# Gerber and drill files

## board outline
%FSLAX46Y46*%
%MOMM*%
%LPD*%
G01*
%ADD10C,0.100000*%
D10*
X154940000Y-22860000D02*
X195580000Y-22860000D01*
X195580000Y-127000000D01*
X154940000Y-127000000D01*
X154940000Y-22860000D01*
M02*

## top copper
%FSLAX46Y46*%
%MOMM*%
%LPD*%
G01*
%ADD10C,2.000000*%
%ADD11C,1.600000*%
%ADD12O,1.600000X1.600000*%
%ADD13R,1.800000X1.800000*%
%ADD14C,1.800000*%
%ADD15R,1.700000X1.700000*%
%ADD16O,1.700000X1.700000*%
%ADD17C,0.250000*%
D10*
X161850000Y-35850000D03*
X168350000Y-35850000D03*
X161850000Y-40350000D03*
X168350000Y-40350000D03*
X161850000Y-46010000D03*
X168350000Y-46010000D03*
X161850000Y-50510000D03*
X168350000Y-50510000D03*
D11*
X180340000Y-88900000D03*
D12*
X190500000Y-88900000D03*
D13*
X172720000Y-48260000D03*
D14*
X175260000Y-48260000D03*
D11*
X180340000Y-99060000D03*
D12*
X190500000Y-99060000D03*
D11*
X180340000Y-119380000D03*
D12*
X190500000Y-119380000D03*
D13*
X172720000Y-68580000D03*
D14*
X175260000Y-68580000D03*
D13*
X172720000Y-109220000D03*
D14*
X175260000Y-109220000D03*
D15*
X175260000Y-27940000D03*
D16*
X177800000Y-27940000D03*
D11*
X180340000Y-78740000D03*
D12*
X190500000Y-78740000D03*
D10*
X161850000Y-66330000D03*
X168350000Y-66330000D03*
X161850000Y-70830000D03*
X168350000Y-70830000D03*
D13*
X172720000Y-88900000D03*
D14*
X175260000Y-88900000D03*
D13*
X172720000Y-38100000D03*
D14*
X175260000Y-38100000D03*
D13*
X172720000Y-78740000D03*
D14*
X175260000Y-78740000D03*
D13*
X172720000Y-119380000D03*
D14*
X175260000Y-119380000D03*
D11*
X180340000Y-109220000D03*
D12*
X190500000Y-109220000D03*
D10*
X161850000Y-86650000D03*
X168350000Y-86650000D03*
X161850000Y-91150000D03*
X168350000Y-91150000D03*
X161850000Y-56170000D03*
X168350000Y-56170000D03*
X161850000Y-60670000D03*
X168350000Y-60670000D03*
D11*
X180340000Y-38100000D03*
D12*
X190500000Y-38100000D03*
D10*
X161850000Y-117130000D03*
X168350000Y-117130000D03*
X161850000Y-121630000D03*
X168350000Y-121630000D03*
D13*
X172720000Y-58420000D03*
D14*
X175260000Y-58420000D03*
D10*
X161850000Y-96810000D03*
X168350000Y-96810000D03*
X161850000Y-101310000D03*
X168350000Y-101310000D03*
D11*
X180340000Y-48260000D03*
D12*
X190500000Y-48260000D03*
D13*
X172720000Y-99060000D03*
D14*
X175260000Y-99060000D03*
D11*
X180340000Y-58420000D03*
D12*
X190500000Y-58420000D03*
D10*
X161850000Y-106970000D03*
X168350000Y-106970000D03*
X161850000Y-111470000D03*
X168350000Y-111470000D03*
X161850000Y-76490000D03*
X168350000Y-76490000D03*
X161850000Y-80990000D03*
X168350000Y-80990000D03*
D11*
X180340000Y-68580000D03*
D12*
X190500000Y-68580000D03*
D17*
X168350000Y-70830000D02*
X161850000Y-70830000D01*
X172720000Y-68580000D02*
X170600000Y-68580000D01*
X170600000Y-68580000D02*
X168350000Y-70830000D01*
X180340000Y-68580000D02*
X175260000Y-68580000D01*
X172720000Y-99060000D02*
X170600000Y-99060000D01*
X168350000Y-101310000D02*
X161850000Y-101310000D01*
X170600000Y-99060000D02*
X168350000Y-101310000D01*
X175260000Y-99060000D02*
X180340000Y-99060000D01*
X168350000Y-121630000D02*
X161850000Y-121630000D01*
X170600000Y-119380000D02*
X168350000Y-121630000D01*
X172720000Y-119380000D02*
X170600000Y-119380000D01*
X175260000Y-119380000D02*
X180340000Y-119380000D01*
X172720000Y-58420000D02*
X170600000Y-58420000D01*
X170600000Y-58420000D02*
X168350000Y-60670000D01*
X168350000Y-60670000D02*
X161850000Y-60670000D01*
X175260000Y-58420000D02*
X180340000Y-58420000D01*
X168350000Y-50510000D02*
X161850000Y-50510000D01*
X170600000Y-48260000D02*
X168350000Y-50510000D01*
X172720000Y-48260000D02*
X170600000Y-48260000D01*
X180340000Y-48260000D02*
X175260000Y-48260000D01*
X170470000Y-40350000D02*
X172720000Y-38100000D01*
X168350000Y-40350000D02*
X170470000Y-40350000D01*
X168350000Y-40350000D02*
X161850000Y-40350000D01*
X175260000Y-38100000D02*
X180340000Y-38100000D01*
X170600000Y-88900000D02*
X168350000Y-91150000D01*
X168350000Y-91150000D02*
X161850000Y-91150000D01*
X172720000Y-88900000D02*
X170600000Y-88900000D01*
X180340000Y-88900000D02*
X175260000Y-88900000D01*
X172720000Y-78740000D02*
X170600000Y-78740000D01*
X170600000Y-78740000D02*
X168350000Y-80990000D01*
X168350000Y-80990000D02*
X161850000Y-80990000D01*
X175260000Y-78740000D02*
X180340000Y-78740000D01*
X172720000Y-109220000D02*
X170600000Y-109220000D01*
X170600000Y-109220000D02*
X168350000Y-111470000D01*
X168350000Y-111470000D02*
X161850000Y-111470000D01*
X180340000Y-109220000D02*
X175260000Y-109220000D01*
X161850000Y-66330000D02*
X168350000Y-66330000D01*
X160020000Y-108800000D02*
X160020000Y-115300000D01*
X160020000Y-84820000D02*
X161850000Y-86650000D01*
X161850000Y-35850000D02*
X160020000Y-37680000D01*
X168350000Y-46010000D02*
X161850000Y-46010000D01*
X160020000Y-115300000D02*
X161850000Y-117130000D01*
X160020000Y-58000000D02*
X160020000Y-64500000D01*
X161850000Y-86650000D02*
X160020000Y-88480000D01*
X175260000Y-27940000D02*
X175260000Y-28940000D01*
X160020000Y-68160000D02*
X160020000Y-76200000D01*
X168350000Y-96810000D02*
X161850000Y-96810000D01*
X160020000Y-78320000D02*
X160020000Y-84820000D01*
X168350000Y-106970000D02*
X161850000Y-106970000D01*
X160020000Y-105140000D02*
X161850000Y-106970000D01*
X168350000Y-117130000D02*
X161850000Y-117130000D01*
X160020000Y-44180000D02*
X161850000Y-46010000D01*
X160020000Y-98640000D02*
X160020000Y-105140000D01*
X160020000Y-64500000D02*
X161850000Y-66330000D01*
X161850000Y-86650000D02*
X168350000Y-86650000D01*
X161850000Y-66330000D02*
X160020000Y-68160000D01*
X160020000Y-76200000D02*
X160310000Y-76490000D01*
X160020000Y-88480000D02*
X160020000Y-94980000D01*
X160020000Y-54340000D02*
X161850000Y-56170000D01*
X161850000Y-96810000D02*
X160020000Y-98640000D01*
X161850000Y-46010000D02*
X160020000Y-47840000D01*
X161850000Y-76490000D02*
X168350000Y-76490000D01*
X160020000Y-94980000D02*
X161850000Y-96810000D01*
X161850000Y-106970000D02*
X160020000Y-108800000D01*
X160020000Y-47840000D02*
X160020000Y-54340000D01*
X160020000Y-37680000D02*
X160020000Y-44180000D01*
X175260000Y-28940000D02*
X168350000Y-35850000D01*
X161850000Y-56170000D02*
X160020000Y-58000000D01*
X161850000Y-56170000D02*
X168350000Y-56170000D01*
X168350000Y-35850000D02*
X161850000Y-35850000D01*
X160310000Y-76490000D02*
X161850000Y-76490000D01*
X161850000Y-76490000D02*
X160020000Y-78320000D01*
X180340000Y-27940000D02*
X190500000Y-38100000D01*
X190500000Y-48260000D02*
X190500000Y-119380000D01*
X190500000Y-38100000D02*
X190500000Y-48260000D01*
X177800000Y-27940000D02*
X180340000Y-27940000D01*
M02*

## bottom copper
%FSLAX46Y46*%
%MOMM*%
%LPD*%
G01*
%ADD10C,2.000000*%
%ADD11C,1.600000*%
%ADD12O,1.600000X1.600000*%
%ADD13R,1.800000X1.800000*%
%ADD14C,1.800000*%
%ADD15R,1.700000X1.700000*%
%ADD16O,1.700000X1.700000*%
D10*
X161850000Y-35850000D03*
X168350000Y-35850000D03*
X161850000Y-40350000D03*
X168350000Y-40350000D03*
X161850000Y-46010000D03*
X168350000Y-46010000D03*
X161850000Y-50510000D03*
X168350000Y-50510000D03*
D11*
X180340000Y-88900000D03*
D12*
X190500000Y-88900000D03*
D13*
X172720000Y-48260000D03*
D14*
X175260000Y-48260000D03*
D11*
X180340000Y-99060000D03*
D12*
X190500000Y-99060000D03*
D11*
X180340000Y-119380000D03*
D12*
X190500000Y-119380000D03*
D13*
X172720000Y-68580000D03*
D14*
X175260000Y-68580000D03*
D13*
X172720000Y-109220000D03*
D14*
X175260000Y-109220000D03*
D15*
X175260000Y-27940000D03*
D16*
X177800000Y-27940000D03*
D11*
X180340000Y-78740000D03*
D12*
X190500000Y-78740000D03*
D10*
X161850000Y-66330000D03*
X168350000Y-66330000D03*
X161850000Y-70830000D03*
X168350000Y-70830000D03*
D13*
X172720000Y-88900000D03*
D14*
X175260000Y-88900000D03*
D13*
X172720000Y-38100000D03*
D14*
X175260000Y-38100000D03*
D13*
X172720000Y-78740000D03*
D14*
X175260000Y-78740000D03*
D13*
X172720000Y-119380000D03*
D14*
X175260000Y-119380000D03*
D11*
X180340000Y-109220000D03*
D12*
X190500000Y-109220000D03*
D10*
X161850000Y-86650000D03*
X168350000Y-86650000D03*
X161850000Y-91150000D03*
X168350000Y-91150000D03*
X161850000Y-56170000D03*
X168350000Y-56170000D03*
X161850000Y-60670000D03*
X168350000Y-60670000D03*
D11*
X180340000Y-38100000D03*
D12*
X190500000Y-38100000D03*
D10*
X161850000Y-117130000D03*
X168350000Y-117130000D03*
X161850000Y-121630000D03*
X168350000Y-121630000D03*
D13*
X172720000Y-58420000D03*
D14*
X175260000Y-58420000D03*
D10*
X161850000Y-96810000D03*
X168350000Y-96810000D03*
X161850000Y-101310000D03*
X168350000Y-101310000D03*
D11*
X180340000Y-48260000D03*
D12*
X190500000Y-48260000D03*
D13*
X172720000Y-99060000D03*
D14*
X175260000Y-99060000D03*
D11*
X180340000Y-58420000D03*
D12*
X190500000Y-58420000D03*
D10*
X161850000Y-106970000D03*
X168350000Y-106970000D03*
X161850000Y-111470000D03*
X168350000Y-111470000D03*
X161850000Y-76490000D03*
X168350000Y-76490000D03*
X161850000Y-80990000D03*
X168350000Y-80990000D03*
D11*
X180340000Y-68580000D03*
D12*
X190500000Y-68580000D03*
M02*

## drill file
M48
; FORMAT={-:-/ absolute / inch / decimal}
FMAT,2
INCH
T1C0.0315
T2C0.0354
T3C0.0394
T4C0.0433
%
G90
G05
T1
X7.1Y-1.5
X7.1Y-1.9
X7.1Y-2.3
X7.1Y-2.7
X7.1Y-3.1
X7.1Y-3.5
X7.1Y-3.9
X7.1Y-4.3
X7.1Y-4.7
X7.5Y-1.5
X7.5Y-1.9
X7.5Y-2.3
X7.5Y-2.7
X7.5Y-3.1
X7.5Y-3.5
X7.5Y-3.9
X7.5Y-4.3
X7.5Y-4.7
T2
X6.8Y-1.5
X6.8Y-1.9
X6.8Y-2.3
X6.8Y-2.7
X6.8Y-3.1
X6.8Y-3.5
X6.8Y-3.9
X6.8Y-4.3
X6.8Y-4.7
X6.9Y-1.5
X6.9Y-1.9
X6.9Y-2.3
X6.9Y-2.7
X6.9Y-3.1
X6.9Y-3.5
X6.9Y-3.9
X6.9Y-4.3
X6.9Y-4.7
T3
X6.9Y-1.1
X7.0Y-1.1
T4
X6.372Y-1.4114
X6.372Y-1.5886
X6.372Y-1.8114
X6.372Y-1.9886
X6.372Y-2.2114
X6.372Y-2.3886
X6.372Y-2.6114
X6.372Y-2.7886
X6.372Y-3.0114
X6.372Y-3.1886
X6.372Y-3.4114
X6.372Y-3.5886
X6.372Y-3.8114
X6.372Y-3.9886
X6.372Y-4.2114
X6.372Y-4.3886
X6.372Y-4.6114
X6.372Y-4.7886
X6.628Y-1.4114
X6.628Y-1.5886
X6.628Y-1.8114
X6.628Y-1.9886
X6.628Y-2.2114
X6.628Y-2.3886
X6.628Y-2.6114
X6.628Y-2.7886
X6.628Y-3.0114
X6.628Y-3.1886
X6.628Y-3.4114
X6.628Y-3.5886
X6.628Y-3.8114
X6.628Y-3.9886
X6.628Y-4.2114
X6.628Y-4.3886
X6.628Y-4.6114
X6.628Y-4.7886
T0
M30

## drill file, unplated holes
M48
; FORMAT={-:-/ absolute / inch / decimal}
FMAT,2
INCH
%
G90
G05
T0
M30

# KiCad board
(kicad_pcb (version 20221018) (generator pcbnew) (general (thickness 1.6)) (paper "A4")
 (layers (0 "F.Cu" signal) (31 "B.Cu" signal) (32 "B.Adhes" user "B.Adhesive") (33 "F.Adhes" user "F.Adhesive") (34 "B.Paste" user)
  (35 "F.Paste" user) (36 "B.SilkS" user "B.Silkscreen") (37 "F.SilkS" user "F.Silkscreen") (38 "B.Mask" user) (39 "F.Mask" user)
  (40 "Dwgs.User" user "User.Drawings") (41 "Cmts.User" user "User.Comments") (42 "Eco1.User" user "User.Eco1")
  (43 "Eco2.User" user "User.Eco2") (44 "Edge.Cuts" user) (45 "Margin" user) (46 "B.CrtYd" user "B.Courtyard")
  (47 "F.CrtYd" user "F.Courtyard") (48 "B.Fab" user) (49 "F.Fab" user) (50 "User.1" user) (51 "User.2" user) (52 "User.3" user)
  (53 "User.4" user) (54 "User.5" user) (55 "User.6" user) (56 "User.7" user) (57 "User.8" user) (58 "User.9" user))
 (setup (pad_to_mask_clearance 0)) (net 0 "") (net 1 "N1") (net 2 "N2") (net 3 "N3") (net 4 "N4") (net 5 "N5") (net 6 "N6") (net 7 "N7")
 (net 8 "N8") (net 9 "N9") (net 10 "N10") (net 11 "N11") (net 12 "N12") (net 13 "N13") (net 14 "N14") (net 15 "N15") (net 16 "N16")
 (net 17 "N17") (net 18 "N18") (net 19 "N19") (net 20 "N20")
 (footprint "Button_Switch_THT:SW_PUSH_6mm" (layer "F.Cu") (at 161.85 35.85)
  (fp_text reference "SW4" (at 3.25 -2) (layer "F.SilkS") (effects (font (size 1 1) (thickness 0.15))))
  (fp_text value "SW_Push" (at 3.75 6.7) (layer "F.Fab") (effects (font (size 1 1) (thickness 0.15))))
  (pad "1" thru_hole circle (at 0 0 90) (size 2 2) (drill 1.1) (layers "*.Cu" "*.Mask") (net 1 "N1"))
  (pad "1" thru_hole circle (at 6.5 0 90) (size 2 2) (drill 1.1) (layers "*.Cu" "*.Mask") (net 1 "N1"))
  (pad "2" thru_hole circle (at 0 4.5 90) (size 2 2) (drill 1.1) (layers "*.Cu" "*.Mask") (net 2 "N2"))
  (pad "2" thru_hole circle (at 6.5 4.5 90) (size 2 2) (drill 1.1) (layers "*.Cu" "*.Mask") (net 2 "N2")))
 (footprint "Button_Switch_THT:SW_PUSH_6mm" (layer "F.Cu") (at 161.85 46.01)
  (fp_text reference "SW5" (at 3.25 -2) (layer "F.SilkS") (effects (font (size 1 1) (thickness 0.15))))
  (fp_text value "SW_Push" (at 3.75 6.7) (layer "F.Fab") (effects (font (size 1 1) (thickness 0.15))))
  (pad "1" thru_hole circle (at 0 0 90) (size 2 2) (drill 1.1) (layers "*.Cu" "*.Mask") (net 1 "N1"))
  (pad "1" thru_hole circle (at 6.5 0 90) (size 2 2) (drill 1.1) (layers "*.Cu" "*.Mask") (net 1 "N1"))
  (pad "2" thru_hole circle (at 0 4.5 90) (size 2 2) (drill 1.1) (layers "*.Cu" "*.Mask") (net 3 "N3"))
  (pad "2" thru_hole circle (at 6.5 4.5 90) (size 2 2) (drill 1.1) (layers "*.Cu" "*.Mask") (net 3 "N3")))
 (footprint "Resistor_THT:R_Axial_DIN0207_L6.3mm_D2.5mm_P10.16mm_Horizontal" (layer "F.Cu") (at 180.34 88.9)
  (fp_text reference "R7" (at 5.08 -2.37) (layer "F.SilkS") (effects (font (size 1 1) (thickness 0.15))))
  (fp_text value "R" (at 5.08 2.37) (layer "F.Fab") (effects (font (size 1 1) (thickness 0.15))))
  (pad "1" thru_hole circle (at 0 0) (size 1.6 1.6) (drill 0.8) (layers "*.Cu" "*.Mask") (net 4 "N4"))
  (pad "2" thru_hole oval (at 10.16 0) (size 1.6 1.6) (drill 0.8) (layers "*.Cu" "*.Mask") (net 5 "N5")))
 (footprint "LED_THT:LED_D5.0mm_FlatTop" (layer "F.Cu") (at 172.72 48.26)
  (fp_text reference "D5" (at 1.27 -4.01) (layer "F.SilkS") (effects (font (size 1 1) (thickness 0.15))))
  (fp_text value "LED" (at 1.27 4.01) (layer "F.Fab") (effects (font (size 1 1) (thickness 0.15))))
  (pad "1" thru_hole rect (at 0 0) (size 1.8 1.8) (drill 0.9) (layers "*.Cu" "*.Mask") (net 3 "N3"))
  (pad "2" thru_hole circle (at 2.54 0) (size 1.8 1.8) (drill 0.9) (layers "*.Cu" "*.Mask") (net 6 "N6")))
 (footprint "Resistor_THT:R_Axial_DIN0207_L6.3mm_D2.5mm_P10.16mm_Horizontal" (layer "F.Cu") (at 180.34 99.06)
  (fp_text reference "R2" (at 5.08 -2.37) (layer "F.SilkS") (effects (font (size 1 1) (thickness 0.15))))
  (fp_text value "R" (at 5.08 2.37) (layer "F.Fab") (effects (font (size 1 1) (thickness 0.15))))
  (pad "1" thru_hole circle (at 0 0) (size 1.6 1.6) (drill 0.8) (layers "*.Cu" "*.Mask") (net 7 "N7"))
  (pad "2" thru_hole oval (at 10.16 0) (size 1.6 1.6) (drill 0.8) (layers "*.Cu" "*.Mask") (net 5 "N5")))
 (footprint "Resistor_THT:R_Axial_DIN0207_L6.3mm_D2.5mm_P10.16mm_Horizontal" (layer "F.Cu") (at 180.34 119.38)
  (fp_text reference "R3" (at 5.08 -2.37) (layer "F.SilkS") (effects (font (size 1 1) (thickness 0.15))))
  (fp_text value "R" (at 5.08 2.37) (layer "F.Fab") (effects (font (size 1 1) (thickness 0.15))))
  (pad "1" thru_hole circle (at 0 0) (size 1.6 1.6) (drill 0.8) (layers "*.Cu" "*.Mask") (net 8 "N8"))
  (pad "2" thru_hole oval (at 10.16 0) (size 1.6 1.6) (drill 0.8) (layers "*.Cu" "*.Mask") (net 5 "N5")))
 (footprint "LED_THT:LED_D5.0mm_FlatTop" (layer "F.Cu") (at 172.72 68.58)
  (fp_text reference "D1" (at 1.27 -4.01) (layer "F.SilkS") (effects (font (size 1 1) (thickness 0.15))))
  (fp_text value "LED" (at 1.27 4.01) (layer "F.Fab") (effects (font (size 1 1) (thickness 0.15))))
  (pad "1" thru_hole rect (at 0 0) (size 1.8 1.8) (drill 0.9) (layers "*.Cu" "*.Mask") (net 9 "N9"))
  (pad "2" thru_hole circle (at 2.54 0) (size 1.8 1.8) (drill 0.9) (layers "*.Cu" "*.Mask") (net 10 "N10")))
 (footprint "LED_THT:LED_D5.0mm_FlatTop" (layer "F.Cu") (at 172.72 109.22)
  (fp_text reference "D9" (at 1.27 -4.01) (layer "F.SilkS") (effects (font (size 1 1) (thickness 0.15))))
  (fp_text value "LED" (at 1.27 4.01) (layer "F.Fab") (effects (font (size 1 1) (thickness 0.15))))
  (pad "1" thru_hole rect (at 0 0) (size 1.8 1.8) (drill 0.9) (layers "*.Cu" "*.Mask") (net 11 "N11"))
  (pad "2" thru_hole circle (at 2.54 0) (size 1.8 1.8) (drill 0.9) (layers "*.Cu" "*.Mask") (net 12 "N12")))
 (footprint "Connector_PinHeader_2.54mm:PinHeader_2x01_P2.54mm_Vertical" (layer "F.Cu") (at 175.26 27.94)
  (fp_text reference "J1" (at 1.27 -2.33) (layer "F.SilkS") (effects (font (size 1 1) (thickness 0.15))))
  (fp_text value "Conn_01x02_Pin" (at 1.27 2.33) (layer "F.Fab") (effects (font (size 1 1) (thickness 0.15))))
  (pad "1" thru_hole rect (at 0 0) (size 1.7 1.7) (drill 1) (layers "*.Cu" "*.Mask") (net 1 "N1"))
  (pad "2" thru_hole oval (at 2.54 0) (size 1.7 1.7) (drill 1) (layers "*.Cu" "*.Mask") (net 5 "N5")))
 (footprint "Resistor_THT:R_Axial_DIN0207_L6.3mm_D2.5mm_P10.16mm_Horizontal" (layer "F.Cu") (at 180.34 78.74)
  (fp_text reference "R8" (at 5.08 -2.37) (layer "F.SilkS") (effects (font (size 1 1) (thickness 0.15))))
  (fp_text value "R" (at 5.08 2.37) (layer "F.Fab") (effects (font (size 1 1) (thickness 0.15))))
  (pad "1" thru_hole circle (at 0 0) (size 1.6 1.6) (drill 0.8) (layers "*.Cu" "*.Mask") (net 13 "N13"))
  (pad "2" thru_hole oval (at 10.16 0) (size 1.6 1.6) (drill 0.8) (layers "*.Cu" "*.Mask") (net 5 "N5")))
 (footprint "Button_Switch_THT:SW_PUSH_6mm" (layer "F.Cu") (at 161.85 66.33)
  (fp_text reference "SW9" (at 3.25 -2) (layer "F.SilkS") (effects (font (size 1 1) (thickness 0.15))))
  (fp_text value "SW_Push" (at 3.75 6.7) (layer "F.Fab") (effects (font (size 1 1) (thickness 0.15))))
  (pad "1" thru_hole circle (at 0 0 90) (size 2 2) (drill 1.1) (layers "*.Cu" "*.Mask") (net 1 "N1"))
  (pad "1" thru_hole circle (at 6.5 0 90) (size 2 2) (drill 1.1) (layers "*.Cu" "*.Mask") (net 1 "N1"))
  (pad "2" thru_hole circle (at 0 4.5 90) (size 2 2) (drill 1.1) (layers "*.Cu" "*.Mask") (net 9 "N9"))
  (pad "2" thru_hole circle (at 6.5 4.5 90) (size 2 2) (drill 1.1) (layers "*.Cu" "*.Mask") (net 9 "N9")))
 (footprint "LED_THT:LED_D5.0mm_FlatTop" (layer "F.Cu") (at 172.72 88.9)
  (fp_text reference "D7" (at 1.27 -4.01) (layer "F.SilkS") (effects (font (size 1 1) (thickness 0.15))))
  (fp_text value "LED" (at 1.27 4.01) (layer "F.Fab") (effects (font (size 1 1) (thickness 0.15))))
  (pad "1" thru_hole rect (at 0 0) (size 1.8 1.8) (drill 0.9) (layers "*.Cu" "*.Mask") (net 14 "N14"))
  (pad "2" thru_hole circle (at 2.54 0) (size 1.8 1.8) (drill 0.9) (layers "*.Cu" "*.Mask") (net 4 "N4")))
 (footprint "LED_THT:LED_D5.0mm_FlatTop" (layer "F.Cu") (at 172.72 38.1)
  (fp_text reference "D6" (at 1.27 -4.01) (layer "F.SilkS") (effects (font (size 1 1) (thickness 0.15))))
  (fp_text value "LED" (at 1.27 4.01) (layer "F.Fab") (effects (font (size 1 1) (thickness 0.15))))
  (pad "1" thru_hole rect (at 0 0) (size 1.8 1.8) (drill 0.9) (layers "*.Cu" "*.Mask") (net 2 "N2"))
  (pad "2" thru_hole circle (at 2.54 0) (size 1.8 1.8) (drill 0.9) (layers "*.Cu" "*.Mask") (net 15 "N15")))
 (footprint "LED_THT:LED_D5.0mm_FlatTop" (layer "F.Cu") (at 172.72 78.74)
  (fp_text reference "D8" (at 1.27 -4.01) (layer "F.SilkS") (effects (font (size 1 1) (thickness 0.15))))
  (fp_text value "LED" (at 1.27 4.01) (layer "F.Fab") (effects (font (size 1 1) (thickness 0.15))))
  (pad "1" thru_hole rect (at 0 0) (size 1.8 1.8) (drill 0.9) (layers "*.Cu" "*.Mask") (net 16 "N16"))
  (pad "2" thru_hole circle (at 2.54 0) (size 1.8 1.8) (drill 0.9) (layers "*.Cu" "*.Mask") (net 13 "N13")))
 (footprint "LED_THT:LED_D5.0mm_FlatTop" (layer "F.Cu") (at 172.72 119.38)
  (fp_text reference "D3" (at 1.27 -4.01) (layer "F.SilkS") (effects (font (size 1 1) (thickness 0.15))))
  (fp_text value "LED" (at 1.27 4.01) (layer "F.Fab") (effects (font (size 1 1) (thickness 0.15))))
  (pad "1" thru_hole rect (at 0 0) (size 1.8 1.8) (drill 0.9) (layers "*.Cu" "*.Mask") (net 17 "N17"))
  (pad "2" thru_hole circle (at 2.54 0) (size 1.8 1.8) (drill 0.9) (layers "*.Cu" "*.Mask") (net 8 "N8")))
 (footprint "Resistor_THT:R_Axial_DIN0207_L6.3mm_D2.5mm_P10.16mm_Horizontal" (layer "F.Cu") (at 180.34 109.22)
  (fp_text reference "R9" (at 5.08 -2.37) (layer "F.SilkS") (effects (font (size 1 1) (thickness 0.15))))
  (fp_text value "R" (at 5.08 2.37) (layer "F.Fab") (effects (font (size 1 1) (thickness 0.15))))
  (pad "1" thru_hole circle (at 0 0) (size 1.6 1.6) (drill 0.8) (layers "*.Cu" "*.Mask") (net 12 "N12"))
  (pad "2" thru_hole oval (at 10.16 0) (size 1.6 1.6) (drill 0.8) (layers "*.Cu" "*.Mask") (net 5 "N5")))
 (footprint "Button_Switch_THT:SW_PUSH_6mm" (layer "F.Cu") (at 161.85 86.65)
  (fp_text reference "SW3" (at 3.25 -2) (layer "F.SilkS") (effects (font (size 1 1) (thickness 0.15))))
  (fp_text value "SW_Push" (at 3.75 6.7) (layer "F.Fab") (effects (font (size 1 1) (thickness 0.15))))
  (pad "1" thru_hole circle (at 0 0 90) (size 2 2) (drill 1.1) (layers "*.Cu" "*.Mask") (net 1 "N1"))
  (pad "1" thru_hole circle (at 6.5 0 90) (size 2 2) (drill 1.1) (layers "*.Cu" "*.Mask") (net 1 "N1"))
  (pad "2" thru_hole circle (at 0 4.5 90) (size 2 2) (drill 1.1) (layers "*.Cu" "*.Mask") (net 14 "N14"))
  (pad "2" thru_hole circle (at 6.5 4.5 90) (size 2 2) (drill 1.1) (layers "*.Cu" "*.Mask") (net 14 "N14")))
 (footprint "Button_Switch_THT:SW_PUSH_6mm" (layer "F.Cu") (at 161.85 56.17)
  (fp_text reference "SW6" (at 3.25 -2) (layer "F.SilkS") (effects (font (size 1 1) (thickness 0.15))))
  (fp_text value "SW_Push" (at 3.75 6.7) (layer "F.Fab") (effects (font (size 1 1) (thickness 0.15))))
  (pad "1" thru_hole circle (at 0 0 90) (size 2 2) (drill 1.1) (layers "*.Cu" "*.Mask") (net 1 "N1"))
  (pad "1" thru_hole circle (at 6.5 0 90) (size 2 2) (drill 1.1) (layers "*.Cu" "*.Mask") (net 1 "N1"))
  (pad "2" thru_hole circle (at 0 4.5 90) (size 2 2) (drill 1.1) (layers "*.Cu" "*.Mask") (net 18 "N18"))
  (pad "2" thru_hole circle (at 6.5 4.5 90) (size 2 2) (drill 1.1) (layers "*.Cu" "*.Mask") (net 18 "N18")))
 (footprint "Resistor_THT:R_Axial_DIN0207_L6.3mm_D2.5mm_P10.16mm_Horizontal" (layer "F.Cu") (at 180.34 38.1)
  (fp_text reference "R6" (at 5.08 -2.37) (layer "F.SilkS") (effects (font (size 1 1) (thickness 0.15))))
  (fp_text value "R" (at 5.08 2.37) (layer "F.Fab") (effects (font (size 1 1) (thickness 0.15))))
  (pad "1" thru_hole circle (at 0 0) (size 1.6 1.6) (drill 0.8) (layers "*.Cu" "*.Mask") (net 15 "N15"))
  (pad "2" thru_hole oval (at 10.16 0) (size 1.6 1.6) (drill 0.8) (layers "*.Cu" "*.Mask") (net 5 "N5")))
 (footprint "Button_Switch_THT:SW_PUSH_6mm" (layer "F.Cu") (at 161.85 117.13)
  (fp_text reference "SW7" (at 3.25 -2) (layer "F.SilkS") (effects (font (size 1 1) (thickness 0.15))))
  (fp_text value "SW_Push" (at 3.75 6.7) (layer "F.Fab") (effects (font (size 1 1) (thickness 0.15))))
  (pad "1" thru_hole circle (at 0 0 90) (size 2 2) (drill 1.1) (layers "*.Cu" "*.Mask") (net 1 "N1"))
  (pad "1" thru_hole circle (at 6.5 0 90) (size 2 2) (drill 1.1) (layers "*.Cu" "*.Mask") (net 1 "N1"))
  (pad "2" thru_hole circle (at 0 4.5 90) (size 2 2) (drill 1.1) (layers "*.Cu" "*.Mask") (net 17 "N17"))
  (pad "2" thru_hole circle (at 6.5 4.5 90) (size 2 2) (drill 1.1) (layers "*.Cu" "*.Mask") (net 17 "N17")))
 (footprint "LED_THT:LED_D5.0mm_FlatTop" (layer "F.Cu") (at 172.72 58.42)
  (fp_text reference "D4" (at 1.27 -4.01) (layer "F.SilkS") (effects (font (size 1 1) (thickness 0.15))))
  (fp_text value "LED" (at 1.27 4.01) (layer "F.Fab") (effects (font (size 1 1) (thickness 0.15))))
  (pad "1" thru_hole rect (at 0 0) (size 1.8 1.8) (drill 0.9) (layers "*.Cu" "*.Mask") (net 18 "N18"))
  (pad "2" thru_hole circle (at 2.54 0) (size 1.8 1.8) (drill 0.9) (layers "*.Cu" "*.Mask") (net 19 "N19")))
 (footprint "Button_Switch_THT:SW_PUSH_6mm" (layer "F.Cu") (at 161.85 96.81)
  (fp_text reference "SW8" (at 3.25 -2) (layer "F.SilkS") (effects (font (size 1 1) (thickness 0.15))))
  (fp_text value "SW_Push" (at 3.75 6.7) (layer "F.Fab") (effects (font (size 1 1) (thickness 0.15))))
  (pad "1" thru_hole circle (at 0 0 90) (size 2 2) (drill 1.1) (layers "*.Cu" "*.Mask") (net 1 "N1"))
  (pad "1" thru_hole circle (at 6.5 0 90) (size 2 2) (drill 1.1) (layers "*.Cu" "*.Mask") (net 1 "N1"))
  (pad "2" thru_hole circle (at 0 4.5 90) (size 2 2) (drill 1.1) (layers "*.Cu" "*.Mask") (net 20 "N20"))
  (pad "2" thru_hole circle (at 6.5 4.5 90) (size 2 2) (drill 1.1) (layers "*.Cu" "*.Mask") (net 20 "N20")))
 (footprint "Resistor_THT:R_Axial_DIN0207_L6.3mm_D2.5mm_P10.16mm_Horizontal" (layer "F.Cu") (at 180.34 48.26)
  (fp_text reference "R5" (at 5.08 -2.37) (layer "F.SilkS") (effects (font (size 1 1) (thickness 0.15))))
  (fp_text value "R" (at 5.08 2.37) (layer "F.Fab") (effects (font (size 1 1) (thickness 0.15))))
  (pad "1" thru_hole circle (at 0 0) (size 1.6 1.6) (drill 0.8) (layers "*.Cu" "*.Mask") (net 6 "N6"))
  (pad "2" thru_hole oval (at 10.16 0) (size 1.6 1.6) (drill 0.8) (layers "*.Cu" "*.Mask") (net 5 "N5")))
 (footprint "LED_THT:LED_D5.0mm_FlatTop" (layer "F.Cu") (at 172.72 99.06)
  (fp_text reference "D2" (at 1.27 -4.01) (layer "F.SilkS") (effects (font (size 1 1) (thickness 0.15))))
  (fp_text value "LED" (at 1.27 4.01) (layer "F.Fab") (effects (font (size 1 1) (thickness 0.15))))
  (pad "1" thru_hole rect (at 0 0) (size 1.8 1.8) (drill 0.9) (layers "*.Cu" "*.Mask") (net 20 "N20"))
  (pad "2" thru_hole circle (at 2.54 0) (size 1.8 1.8) (drill 0.9) (layers "*.Cu" "*.Mask") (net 7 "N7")))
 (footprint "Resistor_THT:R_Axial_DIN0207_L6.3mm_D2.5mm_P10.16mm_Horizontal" (layer "F.Cu") (at 180.34 58.42)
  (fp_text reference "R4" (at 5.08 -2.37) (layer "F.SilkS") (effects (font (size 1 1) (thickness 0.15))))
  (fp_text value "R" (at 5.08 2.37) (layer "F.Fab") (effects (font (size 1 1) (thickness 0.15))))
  (pad "1" thru_hole circle (at 0 0) (size 1.6 1.6) (drill 0.8) (layers "*.Cu" "*.Mask") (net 19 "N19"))
  (pad "2" thru_hole oval (at 10.16 0) (size 1.6 1.6) (drill 0.8) (layers "*.Cu" "*.Mask") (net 5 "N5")))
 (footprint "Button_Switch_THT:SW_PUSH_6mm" (layer "F.Cu") (at 161.85 106.97)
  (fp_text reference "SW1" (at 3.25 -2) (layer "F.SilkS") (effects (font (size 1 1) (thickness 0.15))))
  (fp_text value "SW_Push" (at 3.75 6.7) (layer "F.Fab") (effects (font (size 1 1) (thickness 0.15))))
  (pad "1" thru_hole circle (at 0 0 90) (size 2 2) (drill 1.1) (layers "*.Cu" "*.Mask") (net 1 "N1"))
  (pad "1" thru_hole circle (at 6.5 0 90) (size 2 2) (drill 1.1) (layers "*.Cu" "*.Mask") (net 1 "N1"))
  (pad "2" thru_hole circle (at 0 4.5 90) (size 2 2) (drill 1.1) (layers "*.Cu" "*.Mask") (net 11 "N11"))
  (pad "2" thru_hole circle (at 6.5 4.5 90) (size 2 2) (drill 1.1) (layers "*.Cu" "*.Mask") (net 11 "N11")))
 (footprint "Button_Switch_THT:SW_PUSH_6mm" (layer "F.Cu") (at 161.85 76.49)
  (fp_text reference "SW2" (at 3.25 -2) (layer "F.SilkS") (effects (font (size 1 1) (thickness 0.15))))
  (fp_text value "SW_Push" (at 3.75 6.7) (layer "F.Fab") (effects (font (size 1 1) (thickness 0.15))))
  (pad "1" thru_hole circle (at 0 0 90) (size 2 2) (drill 1.1) (layers "*.Cu" "*.Mask") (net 1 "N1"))
  (pad "1" thru_hole circle (at 6.5 0 90) (size 2 2) (drill 1.1) (layers "*.Cu" "*.Mask") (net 1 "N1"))
  (pad "2" thru_hole circle (at 0 4.5 90) (size 2 2) (drill 1.1) (layers "*.Cu" "*.Mask") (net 16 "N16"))
  (pad "2" thru_hole circle (at 6.5 4.5 90) (size 2 2) (drill 1.1) (layers "*.Cu" "*.Mask") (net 16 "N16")))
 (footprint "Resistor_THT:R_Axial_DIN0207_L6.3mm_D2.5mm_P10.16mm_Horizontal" (layer "F.Cu") (at 180.34 68.58)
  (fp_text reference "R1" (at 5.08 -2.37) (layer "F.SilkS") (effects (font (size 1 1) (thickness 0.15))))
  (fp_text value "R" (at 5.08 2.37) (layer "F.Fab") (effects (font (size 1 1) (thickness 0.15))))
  (pad "1" thru_hole circle (at 0 0) (size 1.6 1.6) (drill 0.8) (layers "*.Cu" "*.Mask") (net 10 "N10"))
  (pad "2" thru_hole oval (at 10.16 0) (size 1.6 1.6) (drill 0.8) (layers "*.Cu" "*.Mask") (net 5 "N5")))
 (gr_rect (start 154.94 22.86) (end 195.58 127) (stroke (width 0.1) (type default)) (fill none) (layer "Edge.Cuts"))
 (segment (start 168.35 70.83) (end 161.85 70.83) (width 0.25) (layer "F.Cu") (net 9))
 (segment (start 172.72 68.58) (end 170.6 68.58) (width 0.25) (layer "F.Cu") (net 9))
 (segment (start 170.6 68.58) (end 168.35 70.83) (width 0.25) (layer "F.Cu") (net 9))
 (segment (start 180.34 68.58) (end 175.26 68.58) (width 0.25) (layer "F.Cu") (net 10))
 (segment (start 172.72 99.06) (end 170.6 99.06) (width 0.25) (layer "F.Cu") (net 20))
 (segment (start 168.35 101.31) (end 161.85 101.31) (width 0.25) (layer "F.Cu") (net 20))
 (segment (start 170.6 99.06) (end 168.35 101.31) (width 0.25) (layer "F.Cu") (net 20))
 (segment (start 175.26 99.06) (end 180.34 99.06) (width 0.25) (layer "F.Cu") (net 7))
 (segment (start 168.35 121.63) (end 161.85 121.63) (width 0.25) (layer "F.Cu") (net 17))
 (segment (start 170.6 119.38) (end 168.35 121.63) (width 0.25) (layer "F.Cu") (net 17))
 (segment (start 172.72 119.38) (end 170.6 119.38) (width 0.25) (layer "F.Cu") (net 17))
 (segment (start 175.26 119.38) (end 180.34 119.38) (width 0.25) (layer "F.Cu") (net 8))
 (segment (start 172.72 58.42) (end 170.6 58.42) (width 0.25) (layer "F.Cu") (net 18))
 (segment (start 170.6 58.42) (end 168.35 60.67) (width 0.25) (layer "F.Cu") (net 18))
 (segment (start 168.35 60.67) (end 161.85 60.67) (width 0.25) (layer "F.Cu") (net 18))
 (segment (start 175.26 58.42) (end 180.34 58.42) (width 0.25) (layer "F.Cu") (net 19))
 (segment (start 168.35 50.51) (end 161.85 50.51) (width 0.25) (layer "F.Cu") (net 3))
 (segment (start 170.6 48.26) (end 168.35 50.51) (width 0.25) (layer "F.Cu") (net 3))
 (segment (start 172.72 48.26) (end 170.6 48.26) (width 0.25) (layer "F.Cu") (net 3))
 (segment (start 180.34 48.26) (end 175.26 48.26) (width 0.25) (layer "F.Cu") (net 6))
 (segment (start 170.47 40.35) (end 172.72 38.1) (width 0.25) (layer "F.Cu") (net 2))
 (segment (start 168.35 40.35) (end 170.47 40.35) (width 0.25) (layer "F.Cu") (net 2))
 (segment (start 168.35 40.35) (end 161.85 40.35) (width 0.25) (layer "F.Cu") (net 2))
 (segment (start 175.26 38.1) (end 180.34 38.1) (width 0.25) (layer "F.Cu") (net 15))
 (segment (start 170.6 88.9) (end 168.35 91.15) (width 0.25) (layer "F.Cu") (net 14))
 (segment (start 168.35 91.15) (end 161.85 91.15) (width 0.25) (layer "F.Cu") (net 14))
 (segment (start 172.72 88.9) (end 170.6 88.9) (width 0.25) (layer "F.Cu") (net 14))
 (segment (start 180.34 88.9) (end 175.26 88.9) (width 0.25) (layer "F.Cu") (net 4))
 (segment (start 172.72 78.74) (end 170.6 78.74) (width 0.25) (layer "F.Cu") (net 16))
 (segment (start 170.6 78.74) (end 168.35 80.99) (width 0.25) (layer "F.Cu") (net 16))
 (segment (start 168.35 80.99) (end 161.85 80.99) (width 0.25) (layer "F.Cu") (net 16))
 (segment (start 175.26 78.74) (end 180.34 78.74) (width 0.25) (layer "F.Cu") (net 13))
 (segment (start 172.72 109.22) (end 170.6 109.22) (width 0.25) (layer "F.Cu") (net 11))
 (segment (start 170.6 109.22) (end 168.35 111.47) (width 0.25) (layer "F.Cu") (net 11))
 (segment (start 168.35 111.47) (end 161.85 111.47) (width 0.25) (layer "F.Cu") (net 11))
 (segment (start 180.34 109.22) (end 175.26 109.22) (width 0.25) (layer "F.Cu") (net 12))
 (segment (start 161.85 66.33) (end 168.35 66.33) (width 0.25) (layer "F.Cu") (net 1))
 (segment (start 160.02 108.8) (end 160.02 115.3) (width 0.25) (layer "F.Cu") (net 1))
 (segment (start 160.02 84.82) (end 161.85 86.65) (width 0.25) (layer "F.Cu") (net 1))
 (segment (start 161.85 35.85) (end 160.02 37.68) (width 0.25) (layer "F.Cu") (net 1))
 (segment (start 168.35 46.01) (end 161.85 46.01) (width 0.25) (layer "F.Cu") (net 1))
 (segment (start 160.02 115.3) (end 161.85 117.13) (width 0.25) (layer "F.Cu") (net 1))
 (segment (start 160.02 58) (end 160.02 64.5) (width 0.25) (layer "F.Cu") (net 1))
 (segment (start 161.85 86.65) (end 160.02 88.48) (width 0.25) (layer "F.Cu") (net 1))
 (segment (start 175.26 27.94) (end 175.26 28.94) (width 0.25) (layer "F.Cu") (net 1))
 (segment (start 160.02 68.16) (end 160.02 76.2) (width 0.25) (layer "F.Cu") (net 1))
 (segment (start 168.35 96.81) (end 161.85 96.81) (width 0.25) (layer "F.Cu") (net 1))
 (segment (start 160.02 78.32) (end 160.02 84.82) (width 0.25) (layer "F.Cu") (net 1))
 (segment (start 168.35 106.97) (end 161.85 106.97) (width 0.25) (layer "F.Cu") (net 1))
 (segment (start 160.02 105.14) (end 161.85 106.97) (width 0.25) (layer "F.Cu") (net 1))
 (segment (start 168.35 117.13) (end 161.85 117.13) (width 0.25) (layer "F.Cu") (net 1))
 (segment (start 160.02 44.18) (end 161.85 46.01) (width 0.25) (layer "F.Cu") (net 1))
 (segment (start 160.02 98.64) (end 160.02 105.14) (width 0.25) (layer "F.Cu") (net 1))
 (segment (start 160.02 64.5) (end 161.85 66.33) (width 0.25) (layer "F.Cu") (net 1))
 (segment (start 161.85 86.65) (end 168.35 86.65) (width 0.25) (layer "F.Cu") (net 1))
 (segment (start 161.85 66.33) (end 160.02 68.16) (width 0.25) (layer "F.Cu") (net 1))
 (segment (start 160.02 76.2) (end 160.31 76.49) (width 0.25) (layer "F.Cu") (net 1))
 (segment (start 160.02 88.48) (end 160.02 94.98) (width 0.25) (layer "F.Cu") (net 1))
 (segment (start 160.02 54.34) (end 161.85 56.17) (width 0.25) (layer "F.Cu") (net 1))
 (segment (start 161.85 96.81) (end 160.02 98.64) (width 0.25) (layer "F.Cu") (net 1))
 (segment (start 161.85 46.01) (end 160.02 47.84) (width 0.25) (layer "F.Cu") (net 1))
 (segment (start 161.85 76.49) (end 168.35 76.49) (width 0.25) (layer "F.Cu") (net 1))
 (segment (start 160.02 94.98) (end 161.85 96.81) (width 0.25) (layer "F.Cu") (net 1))
 (segment (start 161.85 106.97) (end 160.02 108.8) (width 0.25) (layer "F.Cu") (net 1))
 (segment (start 160.02 47.84) (end 160.02 54.34) (width 0.25) (layer "F.Cu") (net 1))
 (segment (start 160.02 37.68) (end 160.02 44.18) (width 0.25) (layer "F.Cu") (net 1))
 (segment (start 175.26 28.94) (end 168.35 35.85) (width 0.25) (layer "F.Cu") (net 1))
 (segment (start 161.85 56.17) (end 160.02 58) (width 0.25) (layer "F.Cu") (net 1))
 (segment (start 161.85 56.17) (end 168.35 56.17) (width 0.25) (layer "F.Cu") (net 1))
 (segment (start 168.35 35.85) (end 161.85 35.85) (width 0.25) (layer "F.Cu") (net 1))
 (segment (start 160.31 76.49) (end 161.85 76.49) (width 0.25) (layer "F.Cu") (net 1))
 (segment (start 161.85 76.49) (end 160.02 78.32) (width 0.25) (layer "F.Cu") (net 1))
 (segment (start 180.34 27.94) (end 190.5 38.1) (width 0.25) (layer "F.Cu") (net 5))
 (segment (start 190.5 48.26) (end 190.5 119.38) (width 0.25) (layer "F.Cu") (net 5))
 (segment (start 190.5 38.1) (end 190.5 48.26) (width 0.25) (layer "F.Cu") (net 5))
 (segment (start 177.8 27.94) (end 180.34 27.94) (width 0.25) (layer "F.Cu") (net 5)))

